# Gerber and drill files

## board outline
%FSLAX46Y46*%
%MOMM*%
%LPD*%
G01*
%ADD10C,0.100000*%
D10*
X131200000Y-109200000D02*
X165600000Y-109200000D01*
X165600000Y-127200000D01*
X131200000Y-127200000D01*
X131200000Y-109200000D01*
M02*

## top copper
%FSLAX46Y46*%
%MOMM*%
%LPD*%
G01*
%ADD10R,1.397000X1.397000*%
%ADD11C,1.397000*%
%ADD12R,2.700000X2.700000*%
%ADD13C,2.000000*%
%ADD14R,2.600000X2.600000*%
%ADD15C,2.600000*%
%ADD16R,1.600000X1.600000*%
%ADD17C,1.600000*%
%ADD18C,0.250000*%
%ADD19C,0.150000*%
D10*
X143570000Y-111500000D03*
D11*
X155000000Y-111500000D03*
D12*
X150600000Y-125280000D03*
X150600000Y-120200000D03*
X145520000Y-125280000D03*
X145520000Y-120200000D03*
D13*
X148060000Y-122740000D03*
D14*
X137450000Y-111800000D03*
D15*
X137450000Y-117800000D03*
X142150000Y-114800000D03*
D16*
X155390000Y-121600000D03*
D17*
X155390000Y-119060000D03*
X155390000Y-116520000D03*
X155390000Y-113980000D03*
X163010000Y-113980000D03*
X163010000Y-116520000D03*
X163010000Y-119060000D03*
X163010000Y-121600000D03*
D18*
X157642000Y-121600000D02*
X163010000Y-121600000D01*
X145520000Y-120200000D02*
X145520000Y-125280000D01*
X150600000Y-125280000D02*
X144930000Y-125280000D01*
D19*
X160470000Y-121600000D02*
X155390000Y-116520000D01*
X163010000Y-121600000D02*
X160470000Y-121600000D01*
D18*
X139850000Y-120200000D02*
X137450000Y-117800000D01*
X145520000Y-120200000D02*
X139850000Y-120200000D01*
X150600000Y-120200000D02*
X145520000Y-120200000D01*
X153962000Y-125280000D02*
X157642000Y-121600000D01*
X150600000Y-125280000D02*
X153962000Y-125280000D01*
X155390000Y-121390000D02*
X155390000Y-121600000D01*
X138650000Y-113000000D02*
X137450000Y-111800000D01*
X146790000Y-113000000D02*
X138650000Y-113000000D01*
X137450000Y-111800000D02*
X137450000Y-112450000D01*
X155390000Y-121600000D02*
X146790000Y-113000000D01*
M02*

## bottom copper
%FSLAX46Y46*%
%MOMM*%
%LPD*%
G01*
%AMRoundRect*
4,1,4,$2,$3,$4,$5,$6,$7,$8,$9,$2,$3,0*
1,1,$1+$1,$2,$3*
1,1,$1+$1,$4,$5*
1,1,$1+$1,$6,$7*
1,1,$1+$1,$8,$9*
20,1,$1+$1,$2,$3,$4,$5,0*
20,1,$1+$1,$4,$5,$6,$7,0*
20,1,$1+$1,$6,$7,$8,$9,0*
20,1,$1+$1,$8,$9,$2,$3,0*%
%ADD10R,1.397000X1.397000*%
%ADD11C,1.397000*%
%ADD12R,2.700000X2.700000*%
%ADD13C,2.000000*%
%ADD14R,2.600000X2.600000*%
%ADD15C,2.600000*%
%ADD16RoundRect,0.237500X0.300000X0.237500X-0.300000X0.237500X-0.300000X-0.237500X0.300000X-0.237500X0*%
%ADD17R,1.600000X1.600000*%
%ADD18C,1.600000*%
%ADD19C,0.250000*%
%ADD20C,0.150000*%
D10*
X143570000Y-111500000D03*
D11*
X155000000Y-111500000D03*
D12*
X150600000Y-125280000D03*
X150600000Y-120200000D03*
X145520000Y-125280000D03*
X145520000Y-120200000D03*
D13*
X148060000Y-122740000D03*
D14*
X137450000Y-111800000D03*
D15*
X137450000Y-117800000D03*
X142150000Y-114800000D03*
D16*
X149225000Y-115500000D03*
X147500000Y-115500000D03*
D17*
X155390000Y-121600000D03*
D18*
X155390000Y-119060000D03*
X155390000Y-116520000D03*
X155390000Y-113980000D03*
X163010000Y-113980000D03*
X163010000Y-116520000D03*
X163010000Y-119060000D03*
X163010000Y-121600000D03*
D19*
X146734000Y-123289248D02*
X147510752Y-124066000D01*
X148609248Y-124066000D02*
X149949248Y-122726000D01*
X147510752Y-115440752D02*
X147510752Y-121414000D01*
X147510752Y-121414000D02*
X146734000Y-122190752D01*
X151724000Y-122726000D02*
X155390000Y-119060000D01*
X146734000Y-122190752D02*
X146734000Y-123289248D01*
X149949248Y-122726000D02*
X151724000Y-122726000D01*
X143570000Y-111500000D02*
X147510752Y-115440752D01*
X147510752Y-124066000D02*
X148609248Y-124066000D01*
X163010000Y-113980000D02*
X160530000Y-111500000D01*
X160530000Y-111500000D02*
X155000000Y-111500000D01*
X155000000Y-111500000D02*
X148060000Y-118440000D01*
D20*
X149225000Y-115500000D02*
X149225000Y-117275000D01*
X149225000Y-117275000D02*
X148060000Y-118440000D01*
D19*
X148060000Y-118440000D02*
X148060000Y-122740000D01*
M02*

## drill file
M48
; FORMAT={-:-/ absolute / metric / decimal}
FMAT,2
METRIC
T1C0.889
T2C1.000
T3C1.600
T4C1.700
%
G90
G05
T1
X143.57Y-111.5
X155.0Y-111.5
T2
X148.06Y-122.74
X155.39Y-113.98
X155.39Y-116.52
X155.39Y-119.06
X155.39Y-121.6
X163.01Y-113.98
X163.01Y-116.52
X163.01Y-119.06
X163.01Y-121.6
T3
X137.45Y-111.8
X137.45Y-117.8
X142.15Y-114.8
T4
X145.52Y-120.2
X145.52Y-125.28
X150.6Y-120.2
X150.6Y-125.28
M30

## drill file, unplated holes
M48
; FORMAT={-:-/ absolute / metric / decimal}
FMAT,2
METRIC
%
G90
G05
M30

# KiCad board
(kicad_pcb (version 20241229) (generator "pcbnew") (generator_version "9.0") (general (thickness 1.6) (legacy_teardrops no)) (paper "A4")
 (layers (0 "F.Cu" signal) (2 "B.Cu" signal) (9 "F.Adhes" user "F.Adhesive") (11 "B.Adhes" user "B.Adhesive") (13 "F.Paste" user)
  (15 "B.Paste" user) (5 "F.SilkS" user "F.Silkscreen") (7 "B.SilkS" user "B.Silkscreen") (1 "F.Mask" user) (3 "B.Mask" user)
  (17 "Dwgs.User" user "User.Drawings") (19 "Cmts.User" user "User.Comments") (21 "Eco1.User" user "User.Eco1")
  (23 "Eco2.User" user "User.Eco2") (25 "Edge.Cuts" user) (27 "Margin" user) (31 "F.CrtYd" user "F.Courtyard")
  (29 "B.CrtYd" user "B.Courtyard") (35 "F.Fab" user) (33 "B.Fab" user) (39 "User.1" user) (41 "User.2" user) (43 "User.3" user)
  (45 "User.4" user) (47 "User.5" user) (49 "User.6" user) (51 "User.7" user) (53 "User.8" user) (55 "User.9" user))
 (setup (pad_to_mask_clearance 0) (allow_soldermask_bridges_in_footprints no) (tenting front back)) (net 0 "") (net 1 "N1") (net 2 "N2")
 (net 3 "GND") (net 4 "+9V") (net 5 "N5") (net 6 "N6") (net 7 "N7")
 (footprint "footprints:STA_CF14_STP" (layer "F.Cu") (at 143.57 111.5)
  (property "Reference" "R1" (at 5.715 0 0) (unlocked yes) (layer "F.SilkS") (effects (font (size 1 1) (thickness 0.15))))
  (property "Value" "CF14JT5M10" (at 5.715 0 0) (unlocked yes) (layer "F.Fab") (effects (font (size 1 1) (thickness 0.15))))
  (pad "1" thru_hole rect (at 0 0) (size 1.397 1.397) (drill 0.889) (layers "*.Cu" "*.Mask") (remove_unused_layers no) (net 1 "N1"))
  (pad "2" thru_hole circle (at 11.43 0) (size 1.397 1.397) (drill 0.889) (layers "*.Cu" "*.Mask") (remove_unused_layers no) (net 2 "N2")))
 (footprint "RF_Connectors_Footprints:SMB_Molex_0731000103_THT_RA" (layer "F.Cu") (at 148.06 122.74 180)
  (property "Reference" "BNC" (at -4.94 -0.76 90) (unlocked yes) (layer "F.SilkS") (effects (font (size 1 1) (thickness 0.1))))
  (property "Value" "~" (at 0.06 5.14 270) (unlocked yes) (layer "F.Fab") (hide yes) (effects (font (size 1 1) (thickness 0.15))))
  (pad "1" thru_hole rect (at -2.54 -2.54 270) (size 2.7 2.7) (drill 1.7) (layers "*.Cu" "*.Mask") (remove_unused_layers no) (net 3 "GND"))
  (pad "1" thru_hole rect (at -2.54 2.54 270) (size 2.7 2.7) (drill 1.7) (layers "*.Cu" "*.Mask") (remove_unused_layers no) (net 3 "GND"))
  (pad "1" thru_hole rect (at 2.54 -2.54 270) (size 2.7 2.7) (drill 1.7) (layers "*.Cu" "*.Mask") (remove_unused_layers no) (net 3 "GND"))
  (pad "1" thru_hole rect (at 2.54 2.54 270) (size 2.7 2.7) (drill 1.7) (layers "*.Cu" "*.Mask") (remove_unused_layers no) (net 3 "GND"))
  (pad "2" thru_hole circle (at 0 0 180) (size 2 2) (drill 1) (layers "*.Cu" "*.Mask") (remove_unused_layers no) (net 2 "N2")))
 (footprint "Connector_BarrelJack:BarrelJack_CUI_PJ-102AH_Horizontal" (layer "F.Cu") (at 137.45 111.8)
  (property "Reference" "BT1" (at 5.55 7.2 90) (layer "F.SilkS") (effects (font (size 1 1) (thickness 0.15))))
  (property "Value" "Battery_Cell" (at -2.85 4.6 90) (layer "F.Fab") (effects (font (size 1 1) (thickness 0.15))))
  (pad "1" thru_hole rect (at 0 0) (size 2.6 2.6) (drill 1.6) (layers "*.Cu" "*.Mask") (remove_unused_layers no) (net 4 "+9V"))
  (pad "2" thru_hole circle (at 0 6) (size 2.6 2.6) (drill 1.6) (layers "*.Cu" "*.Mask") (remove_unused_layers no) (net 3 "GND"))
  (pad "3" thru_hole circle (at 4.7 3) (size 2.6 2.6) (drill 1.6) (layers "*.Cu" "*.Mask") (remove_unused_layers no)))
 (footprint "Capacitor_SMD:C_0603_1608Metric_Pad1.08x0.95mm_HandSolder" (layer "B.Cu") (at 148.3625 115.5 180)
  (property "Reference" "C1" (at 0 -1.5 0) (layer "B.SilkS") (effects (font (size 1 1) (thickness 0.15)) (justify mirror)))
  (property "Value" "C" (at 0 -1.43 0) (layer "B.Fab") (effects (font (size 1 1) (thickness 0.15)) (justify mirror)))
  (pad "1" smd roundrect (at -0.8625 0 180) (size 1.075 0.95) (layers "B.Cu" "B.Mask" "B.Paste") (roundrect_rratio 0.25) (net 2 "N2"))
  (pad "2" smd roundrect (at 0.8625 0 180) (size 1.075 0.95) (layers "B.Cu" "B.Mask" "B.Paste") (roundrect_rratio 0.25) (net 1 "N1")))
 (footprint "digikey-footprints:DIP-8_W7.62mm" (layer "B.Cu") (at 155.39 121.6)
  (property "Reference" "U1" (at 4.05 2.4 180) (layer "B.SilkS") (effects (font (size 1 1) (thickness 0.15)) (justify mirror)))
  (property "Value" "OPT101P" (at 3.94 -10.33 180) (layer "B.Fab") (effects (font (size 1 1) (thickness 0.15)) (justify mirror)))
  (pad "1" thru_hole rect (at 0 0) (size 1.6 1.6) (drill 1) (layers "*.Cu" "*.Mask") (remove_unused_layers no) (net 4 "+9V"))
  (pad "2" thru_hole circle (at 0 -2.54) (size 1.6 1.6) (drill 1) (layers "*.Cu" "*.Mask") (remove_unused_layers no) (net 1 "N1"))
  (pad "3" thru_hole circle (at 0 -5.08) (size 1.6 1.6) (drill 1) (layers "*.Cu" "*.Mask") (remove_unused_layers no) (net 3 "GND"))
  (pad "4" thru_hole circle (at 0 -7.62) (size 1.6 1.6) (drill 1) (layers "*.Cu" "*.Mask") (remove_unused_layers no) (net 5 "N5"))
  (pad "5" thru_hole circle (at 7.62 -7.62) (size 1.6 1.6) (drill 1) (layers "*.Cu" "*.Mask") (remove_unused_layers no) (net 2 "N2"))
  (pad "6" thru_hole circle (at 7.62 -5.08) (size 1.6 1.6) (drill 1) (layers "*.Cu" "*.Mask") (remove_unused_layers no) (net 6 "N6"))
  (pad "7" thru_hole circle (at 7.62 -2.54) (size 1.6 1.6) (drill 1) (layers "*.Cu" "*.Mask") (remove_unused_layers no) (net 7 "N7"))
  (pad "8" thru_hole circle (at 7.62 0) (size 1.6 1.6) (drill 1) (layers "*.Cu" "*.Mask") (remove_unused_layers no) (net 3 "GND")))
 (gr_rect (start 131.2 109.2) (end 165.6 127.2) (stroke (width 0.1) (type default)) (fill no) (locked yes) (layer "Edge.Cuts"))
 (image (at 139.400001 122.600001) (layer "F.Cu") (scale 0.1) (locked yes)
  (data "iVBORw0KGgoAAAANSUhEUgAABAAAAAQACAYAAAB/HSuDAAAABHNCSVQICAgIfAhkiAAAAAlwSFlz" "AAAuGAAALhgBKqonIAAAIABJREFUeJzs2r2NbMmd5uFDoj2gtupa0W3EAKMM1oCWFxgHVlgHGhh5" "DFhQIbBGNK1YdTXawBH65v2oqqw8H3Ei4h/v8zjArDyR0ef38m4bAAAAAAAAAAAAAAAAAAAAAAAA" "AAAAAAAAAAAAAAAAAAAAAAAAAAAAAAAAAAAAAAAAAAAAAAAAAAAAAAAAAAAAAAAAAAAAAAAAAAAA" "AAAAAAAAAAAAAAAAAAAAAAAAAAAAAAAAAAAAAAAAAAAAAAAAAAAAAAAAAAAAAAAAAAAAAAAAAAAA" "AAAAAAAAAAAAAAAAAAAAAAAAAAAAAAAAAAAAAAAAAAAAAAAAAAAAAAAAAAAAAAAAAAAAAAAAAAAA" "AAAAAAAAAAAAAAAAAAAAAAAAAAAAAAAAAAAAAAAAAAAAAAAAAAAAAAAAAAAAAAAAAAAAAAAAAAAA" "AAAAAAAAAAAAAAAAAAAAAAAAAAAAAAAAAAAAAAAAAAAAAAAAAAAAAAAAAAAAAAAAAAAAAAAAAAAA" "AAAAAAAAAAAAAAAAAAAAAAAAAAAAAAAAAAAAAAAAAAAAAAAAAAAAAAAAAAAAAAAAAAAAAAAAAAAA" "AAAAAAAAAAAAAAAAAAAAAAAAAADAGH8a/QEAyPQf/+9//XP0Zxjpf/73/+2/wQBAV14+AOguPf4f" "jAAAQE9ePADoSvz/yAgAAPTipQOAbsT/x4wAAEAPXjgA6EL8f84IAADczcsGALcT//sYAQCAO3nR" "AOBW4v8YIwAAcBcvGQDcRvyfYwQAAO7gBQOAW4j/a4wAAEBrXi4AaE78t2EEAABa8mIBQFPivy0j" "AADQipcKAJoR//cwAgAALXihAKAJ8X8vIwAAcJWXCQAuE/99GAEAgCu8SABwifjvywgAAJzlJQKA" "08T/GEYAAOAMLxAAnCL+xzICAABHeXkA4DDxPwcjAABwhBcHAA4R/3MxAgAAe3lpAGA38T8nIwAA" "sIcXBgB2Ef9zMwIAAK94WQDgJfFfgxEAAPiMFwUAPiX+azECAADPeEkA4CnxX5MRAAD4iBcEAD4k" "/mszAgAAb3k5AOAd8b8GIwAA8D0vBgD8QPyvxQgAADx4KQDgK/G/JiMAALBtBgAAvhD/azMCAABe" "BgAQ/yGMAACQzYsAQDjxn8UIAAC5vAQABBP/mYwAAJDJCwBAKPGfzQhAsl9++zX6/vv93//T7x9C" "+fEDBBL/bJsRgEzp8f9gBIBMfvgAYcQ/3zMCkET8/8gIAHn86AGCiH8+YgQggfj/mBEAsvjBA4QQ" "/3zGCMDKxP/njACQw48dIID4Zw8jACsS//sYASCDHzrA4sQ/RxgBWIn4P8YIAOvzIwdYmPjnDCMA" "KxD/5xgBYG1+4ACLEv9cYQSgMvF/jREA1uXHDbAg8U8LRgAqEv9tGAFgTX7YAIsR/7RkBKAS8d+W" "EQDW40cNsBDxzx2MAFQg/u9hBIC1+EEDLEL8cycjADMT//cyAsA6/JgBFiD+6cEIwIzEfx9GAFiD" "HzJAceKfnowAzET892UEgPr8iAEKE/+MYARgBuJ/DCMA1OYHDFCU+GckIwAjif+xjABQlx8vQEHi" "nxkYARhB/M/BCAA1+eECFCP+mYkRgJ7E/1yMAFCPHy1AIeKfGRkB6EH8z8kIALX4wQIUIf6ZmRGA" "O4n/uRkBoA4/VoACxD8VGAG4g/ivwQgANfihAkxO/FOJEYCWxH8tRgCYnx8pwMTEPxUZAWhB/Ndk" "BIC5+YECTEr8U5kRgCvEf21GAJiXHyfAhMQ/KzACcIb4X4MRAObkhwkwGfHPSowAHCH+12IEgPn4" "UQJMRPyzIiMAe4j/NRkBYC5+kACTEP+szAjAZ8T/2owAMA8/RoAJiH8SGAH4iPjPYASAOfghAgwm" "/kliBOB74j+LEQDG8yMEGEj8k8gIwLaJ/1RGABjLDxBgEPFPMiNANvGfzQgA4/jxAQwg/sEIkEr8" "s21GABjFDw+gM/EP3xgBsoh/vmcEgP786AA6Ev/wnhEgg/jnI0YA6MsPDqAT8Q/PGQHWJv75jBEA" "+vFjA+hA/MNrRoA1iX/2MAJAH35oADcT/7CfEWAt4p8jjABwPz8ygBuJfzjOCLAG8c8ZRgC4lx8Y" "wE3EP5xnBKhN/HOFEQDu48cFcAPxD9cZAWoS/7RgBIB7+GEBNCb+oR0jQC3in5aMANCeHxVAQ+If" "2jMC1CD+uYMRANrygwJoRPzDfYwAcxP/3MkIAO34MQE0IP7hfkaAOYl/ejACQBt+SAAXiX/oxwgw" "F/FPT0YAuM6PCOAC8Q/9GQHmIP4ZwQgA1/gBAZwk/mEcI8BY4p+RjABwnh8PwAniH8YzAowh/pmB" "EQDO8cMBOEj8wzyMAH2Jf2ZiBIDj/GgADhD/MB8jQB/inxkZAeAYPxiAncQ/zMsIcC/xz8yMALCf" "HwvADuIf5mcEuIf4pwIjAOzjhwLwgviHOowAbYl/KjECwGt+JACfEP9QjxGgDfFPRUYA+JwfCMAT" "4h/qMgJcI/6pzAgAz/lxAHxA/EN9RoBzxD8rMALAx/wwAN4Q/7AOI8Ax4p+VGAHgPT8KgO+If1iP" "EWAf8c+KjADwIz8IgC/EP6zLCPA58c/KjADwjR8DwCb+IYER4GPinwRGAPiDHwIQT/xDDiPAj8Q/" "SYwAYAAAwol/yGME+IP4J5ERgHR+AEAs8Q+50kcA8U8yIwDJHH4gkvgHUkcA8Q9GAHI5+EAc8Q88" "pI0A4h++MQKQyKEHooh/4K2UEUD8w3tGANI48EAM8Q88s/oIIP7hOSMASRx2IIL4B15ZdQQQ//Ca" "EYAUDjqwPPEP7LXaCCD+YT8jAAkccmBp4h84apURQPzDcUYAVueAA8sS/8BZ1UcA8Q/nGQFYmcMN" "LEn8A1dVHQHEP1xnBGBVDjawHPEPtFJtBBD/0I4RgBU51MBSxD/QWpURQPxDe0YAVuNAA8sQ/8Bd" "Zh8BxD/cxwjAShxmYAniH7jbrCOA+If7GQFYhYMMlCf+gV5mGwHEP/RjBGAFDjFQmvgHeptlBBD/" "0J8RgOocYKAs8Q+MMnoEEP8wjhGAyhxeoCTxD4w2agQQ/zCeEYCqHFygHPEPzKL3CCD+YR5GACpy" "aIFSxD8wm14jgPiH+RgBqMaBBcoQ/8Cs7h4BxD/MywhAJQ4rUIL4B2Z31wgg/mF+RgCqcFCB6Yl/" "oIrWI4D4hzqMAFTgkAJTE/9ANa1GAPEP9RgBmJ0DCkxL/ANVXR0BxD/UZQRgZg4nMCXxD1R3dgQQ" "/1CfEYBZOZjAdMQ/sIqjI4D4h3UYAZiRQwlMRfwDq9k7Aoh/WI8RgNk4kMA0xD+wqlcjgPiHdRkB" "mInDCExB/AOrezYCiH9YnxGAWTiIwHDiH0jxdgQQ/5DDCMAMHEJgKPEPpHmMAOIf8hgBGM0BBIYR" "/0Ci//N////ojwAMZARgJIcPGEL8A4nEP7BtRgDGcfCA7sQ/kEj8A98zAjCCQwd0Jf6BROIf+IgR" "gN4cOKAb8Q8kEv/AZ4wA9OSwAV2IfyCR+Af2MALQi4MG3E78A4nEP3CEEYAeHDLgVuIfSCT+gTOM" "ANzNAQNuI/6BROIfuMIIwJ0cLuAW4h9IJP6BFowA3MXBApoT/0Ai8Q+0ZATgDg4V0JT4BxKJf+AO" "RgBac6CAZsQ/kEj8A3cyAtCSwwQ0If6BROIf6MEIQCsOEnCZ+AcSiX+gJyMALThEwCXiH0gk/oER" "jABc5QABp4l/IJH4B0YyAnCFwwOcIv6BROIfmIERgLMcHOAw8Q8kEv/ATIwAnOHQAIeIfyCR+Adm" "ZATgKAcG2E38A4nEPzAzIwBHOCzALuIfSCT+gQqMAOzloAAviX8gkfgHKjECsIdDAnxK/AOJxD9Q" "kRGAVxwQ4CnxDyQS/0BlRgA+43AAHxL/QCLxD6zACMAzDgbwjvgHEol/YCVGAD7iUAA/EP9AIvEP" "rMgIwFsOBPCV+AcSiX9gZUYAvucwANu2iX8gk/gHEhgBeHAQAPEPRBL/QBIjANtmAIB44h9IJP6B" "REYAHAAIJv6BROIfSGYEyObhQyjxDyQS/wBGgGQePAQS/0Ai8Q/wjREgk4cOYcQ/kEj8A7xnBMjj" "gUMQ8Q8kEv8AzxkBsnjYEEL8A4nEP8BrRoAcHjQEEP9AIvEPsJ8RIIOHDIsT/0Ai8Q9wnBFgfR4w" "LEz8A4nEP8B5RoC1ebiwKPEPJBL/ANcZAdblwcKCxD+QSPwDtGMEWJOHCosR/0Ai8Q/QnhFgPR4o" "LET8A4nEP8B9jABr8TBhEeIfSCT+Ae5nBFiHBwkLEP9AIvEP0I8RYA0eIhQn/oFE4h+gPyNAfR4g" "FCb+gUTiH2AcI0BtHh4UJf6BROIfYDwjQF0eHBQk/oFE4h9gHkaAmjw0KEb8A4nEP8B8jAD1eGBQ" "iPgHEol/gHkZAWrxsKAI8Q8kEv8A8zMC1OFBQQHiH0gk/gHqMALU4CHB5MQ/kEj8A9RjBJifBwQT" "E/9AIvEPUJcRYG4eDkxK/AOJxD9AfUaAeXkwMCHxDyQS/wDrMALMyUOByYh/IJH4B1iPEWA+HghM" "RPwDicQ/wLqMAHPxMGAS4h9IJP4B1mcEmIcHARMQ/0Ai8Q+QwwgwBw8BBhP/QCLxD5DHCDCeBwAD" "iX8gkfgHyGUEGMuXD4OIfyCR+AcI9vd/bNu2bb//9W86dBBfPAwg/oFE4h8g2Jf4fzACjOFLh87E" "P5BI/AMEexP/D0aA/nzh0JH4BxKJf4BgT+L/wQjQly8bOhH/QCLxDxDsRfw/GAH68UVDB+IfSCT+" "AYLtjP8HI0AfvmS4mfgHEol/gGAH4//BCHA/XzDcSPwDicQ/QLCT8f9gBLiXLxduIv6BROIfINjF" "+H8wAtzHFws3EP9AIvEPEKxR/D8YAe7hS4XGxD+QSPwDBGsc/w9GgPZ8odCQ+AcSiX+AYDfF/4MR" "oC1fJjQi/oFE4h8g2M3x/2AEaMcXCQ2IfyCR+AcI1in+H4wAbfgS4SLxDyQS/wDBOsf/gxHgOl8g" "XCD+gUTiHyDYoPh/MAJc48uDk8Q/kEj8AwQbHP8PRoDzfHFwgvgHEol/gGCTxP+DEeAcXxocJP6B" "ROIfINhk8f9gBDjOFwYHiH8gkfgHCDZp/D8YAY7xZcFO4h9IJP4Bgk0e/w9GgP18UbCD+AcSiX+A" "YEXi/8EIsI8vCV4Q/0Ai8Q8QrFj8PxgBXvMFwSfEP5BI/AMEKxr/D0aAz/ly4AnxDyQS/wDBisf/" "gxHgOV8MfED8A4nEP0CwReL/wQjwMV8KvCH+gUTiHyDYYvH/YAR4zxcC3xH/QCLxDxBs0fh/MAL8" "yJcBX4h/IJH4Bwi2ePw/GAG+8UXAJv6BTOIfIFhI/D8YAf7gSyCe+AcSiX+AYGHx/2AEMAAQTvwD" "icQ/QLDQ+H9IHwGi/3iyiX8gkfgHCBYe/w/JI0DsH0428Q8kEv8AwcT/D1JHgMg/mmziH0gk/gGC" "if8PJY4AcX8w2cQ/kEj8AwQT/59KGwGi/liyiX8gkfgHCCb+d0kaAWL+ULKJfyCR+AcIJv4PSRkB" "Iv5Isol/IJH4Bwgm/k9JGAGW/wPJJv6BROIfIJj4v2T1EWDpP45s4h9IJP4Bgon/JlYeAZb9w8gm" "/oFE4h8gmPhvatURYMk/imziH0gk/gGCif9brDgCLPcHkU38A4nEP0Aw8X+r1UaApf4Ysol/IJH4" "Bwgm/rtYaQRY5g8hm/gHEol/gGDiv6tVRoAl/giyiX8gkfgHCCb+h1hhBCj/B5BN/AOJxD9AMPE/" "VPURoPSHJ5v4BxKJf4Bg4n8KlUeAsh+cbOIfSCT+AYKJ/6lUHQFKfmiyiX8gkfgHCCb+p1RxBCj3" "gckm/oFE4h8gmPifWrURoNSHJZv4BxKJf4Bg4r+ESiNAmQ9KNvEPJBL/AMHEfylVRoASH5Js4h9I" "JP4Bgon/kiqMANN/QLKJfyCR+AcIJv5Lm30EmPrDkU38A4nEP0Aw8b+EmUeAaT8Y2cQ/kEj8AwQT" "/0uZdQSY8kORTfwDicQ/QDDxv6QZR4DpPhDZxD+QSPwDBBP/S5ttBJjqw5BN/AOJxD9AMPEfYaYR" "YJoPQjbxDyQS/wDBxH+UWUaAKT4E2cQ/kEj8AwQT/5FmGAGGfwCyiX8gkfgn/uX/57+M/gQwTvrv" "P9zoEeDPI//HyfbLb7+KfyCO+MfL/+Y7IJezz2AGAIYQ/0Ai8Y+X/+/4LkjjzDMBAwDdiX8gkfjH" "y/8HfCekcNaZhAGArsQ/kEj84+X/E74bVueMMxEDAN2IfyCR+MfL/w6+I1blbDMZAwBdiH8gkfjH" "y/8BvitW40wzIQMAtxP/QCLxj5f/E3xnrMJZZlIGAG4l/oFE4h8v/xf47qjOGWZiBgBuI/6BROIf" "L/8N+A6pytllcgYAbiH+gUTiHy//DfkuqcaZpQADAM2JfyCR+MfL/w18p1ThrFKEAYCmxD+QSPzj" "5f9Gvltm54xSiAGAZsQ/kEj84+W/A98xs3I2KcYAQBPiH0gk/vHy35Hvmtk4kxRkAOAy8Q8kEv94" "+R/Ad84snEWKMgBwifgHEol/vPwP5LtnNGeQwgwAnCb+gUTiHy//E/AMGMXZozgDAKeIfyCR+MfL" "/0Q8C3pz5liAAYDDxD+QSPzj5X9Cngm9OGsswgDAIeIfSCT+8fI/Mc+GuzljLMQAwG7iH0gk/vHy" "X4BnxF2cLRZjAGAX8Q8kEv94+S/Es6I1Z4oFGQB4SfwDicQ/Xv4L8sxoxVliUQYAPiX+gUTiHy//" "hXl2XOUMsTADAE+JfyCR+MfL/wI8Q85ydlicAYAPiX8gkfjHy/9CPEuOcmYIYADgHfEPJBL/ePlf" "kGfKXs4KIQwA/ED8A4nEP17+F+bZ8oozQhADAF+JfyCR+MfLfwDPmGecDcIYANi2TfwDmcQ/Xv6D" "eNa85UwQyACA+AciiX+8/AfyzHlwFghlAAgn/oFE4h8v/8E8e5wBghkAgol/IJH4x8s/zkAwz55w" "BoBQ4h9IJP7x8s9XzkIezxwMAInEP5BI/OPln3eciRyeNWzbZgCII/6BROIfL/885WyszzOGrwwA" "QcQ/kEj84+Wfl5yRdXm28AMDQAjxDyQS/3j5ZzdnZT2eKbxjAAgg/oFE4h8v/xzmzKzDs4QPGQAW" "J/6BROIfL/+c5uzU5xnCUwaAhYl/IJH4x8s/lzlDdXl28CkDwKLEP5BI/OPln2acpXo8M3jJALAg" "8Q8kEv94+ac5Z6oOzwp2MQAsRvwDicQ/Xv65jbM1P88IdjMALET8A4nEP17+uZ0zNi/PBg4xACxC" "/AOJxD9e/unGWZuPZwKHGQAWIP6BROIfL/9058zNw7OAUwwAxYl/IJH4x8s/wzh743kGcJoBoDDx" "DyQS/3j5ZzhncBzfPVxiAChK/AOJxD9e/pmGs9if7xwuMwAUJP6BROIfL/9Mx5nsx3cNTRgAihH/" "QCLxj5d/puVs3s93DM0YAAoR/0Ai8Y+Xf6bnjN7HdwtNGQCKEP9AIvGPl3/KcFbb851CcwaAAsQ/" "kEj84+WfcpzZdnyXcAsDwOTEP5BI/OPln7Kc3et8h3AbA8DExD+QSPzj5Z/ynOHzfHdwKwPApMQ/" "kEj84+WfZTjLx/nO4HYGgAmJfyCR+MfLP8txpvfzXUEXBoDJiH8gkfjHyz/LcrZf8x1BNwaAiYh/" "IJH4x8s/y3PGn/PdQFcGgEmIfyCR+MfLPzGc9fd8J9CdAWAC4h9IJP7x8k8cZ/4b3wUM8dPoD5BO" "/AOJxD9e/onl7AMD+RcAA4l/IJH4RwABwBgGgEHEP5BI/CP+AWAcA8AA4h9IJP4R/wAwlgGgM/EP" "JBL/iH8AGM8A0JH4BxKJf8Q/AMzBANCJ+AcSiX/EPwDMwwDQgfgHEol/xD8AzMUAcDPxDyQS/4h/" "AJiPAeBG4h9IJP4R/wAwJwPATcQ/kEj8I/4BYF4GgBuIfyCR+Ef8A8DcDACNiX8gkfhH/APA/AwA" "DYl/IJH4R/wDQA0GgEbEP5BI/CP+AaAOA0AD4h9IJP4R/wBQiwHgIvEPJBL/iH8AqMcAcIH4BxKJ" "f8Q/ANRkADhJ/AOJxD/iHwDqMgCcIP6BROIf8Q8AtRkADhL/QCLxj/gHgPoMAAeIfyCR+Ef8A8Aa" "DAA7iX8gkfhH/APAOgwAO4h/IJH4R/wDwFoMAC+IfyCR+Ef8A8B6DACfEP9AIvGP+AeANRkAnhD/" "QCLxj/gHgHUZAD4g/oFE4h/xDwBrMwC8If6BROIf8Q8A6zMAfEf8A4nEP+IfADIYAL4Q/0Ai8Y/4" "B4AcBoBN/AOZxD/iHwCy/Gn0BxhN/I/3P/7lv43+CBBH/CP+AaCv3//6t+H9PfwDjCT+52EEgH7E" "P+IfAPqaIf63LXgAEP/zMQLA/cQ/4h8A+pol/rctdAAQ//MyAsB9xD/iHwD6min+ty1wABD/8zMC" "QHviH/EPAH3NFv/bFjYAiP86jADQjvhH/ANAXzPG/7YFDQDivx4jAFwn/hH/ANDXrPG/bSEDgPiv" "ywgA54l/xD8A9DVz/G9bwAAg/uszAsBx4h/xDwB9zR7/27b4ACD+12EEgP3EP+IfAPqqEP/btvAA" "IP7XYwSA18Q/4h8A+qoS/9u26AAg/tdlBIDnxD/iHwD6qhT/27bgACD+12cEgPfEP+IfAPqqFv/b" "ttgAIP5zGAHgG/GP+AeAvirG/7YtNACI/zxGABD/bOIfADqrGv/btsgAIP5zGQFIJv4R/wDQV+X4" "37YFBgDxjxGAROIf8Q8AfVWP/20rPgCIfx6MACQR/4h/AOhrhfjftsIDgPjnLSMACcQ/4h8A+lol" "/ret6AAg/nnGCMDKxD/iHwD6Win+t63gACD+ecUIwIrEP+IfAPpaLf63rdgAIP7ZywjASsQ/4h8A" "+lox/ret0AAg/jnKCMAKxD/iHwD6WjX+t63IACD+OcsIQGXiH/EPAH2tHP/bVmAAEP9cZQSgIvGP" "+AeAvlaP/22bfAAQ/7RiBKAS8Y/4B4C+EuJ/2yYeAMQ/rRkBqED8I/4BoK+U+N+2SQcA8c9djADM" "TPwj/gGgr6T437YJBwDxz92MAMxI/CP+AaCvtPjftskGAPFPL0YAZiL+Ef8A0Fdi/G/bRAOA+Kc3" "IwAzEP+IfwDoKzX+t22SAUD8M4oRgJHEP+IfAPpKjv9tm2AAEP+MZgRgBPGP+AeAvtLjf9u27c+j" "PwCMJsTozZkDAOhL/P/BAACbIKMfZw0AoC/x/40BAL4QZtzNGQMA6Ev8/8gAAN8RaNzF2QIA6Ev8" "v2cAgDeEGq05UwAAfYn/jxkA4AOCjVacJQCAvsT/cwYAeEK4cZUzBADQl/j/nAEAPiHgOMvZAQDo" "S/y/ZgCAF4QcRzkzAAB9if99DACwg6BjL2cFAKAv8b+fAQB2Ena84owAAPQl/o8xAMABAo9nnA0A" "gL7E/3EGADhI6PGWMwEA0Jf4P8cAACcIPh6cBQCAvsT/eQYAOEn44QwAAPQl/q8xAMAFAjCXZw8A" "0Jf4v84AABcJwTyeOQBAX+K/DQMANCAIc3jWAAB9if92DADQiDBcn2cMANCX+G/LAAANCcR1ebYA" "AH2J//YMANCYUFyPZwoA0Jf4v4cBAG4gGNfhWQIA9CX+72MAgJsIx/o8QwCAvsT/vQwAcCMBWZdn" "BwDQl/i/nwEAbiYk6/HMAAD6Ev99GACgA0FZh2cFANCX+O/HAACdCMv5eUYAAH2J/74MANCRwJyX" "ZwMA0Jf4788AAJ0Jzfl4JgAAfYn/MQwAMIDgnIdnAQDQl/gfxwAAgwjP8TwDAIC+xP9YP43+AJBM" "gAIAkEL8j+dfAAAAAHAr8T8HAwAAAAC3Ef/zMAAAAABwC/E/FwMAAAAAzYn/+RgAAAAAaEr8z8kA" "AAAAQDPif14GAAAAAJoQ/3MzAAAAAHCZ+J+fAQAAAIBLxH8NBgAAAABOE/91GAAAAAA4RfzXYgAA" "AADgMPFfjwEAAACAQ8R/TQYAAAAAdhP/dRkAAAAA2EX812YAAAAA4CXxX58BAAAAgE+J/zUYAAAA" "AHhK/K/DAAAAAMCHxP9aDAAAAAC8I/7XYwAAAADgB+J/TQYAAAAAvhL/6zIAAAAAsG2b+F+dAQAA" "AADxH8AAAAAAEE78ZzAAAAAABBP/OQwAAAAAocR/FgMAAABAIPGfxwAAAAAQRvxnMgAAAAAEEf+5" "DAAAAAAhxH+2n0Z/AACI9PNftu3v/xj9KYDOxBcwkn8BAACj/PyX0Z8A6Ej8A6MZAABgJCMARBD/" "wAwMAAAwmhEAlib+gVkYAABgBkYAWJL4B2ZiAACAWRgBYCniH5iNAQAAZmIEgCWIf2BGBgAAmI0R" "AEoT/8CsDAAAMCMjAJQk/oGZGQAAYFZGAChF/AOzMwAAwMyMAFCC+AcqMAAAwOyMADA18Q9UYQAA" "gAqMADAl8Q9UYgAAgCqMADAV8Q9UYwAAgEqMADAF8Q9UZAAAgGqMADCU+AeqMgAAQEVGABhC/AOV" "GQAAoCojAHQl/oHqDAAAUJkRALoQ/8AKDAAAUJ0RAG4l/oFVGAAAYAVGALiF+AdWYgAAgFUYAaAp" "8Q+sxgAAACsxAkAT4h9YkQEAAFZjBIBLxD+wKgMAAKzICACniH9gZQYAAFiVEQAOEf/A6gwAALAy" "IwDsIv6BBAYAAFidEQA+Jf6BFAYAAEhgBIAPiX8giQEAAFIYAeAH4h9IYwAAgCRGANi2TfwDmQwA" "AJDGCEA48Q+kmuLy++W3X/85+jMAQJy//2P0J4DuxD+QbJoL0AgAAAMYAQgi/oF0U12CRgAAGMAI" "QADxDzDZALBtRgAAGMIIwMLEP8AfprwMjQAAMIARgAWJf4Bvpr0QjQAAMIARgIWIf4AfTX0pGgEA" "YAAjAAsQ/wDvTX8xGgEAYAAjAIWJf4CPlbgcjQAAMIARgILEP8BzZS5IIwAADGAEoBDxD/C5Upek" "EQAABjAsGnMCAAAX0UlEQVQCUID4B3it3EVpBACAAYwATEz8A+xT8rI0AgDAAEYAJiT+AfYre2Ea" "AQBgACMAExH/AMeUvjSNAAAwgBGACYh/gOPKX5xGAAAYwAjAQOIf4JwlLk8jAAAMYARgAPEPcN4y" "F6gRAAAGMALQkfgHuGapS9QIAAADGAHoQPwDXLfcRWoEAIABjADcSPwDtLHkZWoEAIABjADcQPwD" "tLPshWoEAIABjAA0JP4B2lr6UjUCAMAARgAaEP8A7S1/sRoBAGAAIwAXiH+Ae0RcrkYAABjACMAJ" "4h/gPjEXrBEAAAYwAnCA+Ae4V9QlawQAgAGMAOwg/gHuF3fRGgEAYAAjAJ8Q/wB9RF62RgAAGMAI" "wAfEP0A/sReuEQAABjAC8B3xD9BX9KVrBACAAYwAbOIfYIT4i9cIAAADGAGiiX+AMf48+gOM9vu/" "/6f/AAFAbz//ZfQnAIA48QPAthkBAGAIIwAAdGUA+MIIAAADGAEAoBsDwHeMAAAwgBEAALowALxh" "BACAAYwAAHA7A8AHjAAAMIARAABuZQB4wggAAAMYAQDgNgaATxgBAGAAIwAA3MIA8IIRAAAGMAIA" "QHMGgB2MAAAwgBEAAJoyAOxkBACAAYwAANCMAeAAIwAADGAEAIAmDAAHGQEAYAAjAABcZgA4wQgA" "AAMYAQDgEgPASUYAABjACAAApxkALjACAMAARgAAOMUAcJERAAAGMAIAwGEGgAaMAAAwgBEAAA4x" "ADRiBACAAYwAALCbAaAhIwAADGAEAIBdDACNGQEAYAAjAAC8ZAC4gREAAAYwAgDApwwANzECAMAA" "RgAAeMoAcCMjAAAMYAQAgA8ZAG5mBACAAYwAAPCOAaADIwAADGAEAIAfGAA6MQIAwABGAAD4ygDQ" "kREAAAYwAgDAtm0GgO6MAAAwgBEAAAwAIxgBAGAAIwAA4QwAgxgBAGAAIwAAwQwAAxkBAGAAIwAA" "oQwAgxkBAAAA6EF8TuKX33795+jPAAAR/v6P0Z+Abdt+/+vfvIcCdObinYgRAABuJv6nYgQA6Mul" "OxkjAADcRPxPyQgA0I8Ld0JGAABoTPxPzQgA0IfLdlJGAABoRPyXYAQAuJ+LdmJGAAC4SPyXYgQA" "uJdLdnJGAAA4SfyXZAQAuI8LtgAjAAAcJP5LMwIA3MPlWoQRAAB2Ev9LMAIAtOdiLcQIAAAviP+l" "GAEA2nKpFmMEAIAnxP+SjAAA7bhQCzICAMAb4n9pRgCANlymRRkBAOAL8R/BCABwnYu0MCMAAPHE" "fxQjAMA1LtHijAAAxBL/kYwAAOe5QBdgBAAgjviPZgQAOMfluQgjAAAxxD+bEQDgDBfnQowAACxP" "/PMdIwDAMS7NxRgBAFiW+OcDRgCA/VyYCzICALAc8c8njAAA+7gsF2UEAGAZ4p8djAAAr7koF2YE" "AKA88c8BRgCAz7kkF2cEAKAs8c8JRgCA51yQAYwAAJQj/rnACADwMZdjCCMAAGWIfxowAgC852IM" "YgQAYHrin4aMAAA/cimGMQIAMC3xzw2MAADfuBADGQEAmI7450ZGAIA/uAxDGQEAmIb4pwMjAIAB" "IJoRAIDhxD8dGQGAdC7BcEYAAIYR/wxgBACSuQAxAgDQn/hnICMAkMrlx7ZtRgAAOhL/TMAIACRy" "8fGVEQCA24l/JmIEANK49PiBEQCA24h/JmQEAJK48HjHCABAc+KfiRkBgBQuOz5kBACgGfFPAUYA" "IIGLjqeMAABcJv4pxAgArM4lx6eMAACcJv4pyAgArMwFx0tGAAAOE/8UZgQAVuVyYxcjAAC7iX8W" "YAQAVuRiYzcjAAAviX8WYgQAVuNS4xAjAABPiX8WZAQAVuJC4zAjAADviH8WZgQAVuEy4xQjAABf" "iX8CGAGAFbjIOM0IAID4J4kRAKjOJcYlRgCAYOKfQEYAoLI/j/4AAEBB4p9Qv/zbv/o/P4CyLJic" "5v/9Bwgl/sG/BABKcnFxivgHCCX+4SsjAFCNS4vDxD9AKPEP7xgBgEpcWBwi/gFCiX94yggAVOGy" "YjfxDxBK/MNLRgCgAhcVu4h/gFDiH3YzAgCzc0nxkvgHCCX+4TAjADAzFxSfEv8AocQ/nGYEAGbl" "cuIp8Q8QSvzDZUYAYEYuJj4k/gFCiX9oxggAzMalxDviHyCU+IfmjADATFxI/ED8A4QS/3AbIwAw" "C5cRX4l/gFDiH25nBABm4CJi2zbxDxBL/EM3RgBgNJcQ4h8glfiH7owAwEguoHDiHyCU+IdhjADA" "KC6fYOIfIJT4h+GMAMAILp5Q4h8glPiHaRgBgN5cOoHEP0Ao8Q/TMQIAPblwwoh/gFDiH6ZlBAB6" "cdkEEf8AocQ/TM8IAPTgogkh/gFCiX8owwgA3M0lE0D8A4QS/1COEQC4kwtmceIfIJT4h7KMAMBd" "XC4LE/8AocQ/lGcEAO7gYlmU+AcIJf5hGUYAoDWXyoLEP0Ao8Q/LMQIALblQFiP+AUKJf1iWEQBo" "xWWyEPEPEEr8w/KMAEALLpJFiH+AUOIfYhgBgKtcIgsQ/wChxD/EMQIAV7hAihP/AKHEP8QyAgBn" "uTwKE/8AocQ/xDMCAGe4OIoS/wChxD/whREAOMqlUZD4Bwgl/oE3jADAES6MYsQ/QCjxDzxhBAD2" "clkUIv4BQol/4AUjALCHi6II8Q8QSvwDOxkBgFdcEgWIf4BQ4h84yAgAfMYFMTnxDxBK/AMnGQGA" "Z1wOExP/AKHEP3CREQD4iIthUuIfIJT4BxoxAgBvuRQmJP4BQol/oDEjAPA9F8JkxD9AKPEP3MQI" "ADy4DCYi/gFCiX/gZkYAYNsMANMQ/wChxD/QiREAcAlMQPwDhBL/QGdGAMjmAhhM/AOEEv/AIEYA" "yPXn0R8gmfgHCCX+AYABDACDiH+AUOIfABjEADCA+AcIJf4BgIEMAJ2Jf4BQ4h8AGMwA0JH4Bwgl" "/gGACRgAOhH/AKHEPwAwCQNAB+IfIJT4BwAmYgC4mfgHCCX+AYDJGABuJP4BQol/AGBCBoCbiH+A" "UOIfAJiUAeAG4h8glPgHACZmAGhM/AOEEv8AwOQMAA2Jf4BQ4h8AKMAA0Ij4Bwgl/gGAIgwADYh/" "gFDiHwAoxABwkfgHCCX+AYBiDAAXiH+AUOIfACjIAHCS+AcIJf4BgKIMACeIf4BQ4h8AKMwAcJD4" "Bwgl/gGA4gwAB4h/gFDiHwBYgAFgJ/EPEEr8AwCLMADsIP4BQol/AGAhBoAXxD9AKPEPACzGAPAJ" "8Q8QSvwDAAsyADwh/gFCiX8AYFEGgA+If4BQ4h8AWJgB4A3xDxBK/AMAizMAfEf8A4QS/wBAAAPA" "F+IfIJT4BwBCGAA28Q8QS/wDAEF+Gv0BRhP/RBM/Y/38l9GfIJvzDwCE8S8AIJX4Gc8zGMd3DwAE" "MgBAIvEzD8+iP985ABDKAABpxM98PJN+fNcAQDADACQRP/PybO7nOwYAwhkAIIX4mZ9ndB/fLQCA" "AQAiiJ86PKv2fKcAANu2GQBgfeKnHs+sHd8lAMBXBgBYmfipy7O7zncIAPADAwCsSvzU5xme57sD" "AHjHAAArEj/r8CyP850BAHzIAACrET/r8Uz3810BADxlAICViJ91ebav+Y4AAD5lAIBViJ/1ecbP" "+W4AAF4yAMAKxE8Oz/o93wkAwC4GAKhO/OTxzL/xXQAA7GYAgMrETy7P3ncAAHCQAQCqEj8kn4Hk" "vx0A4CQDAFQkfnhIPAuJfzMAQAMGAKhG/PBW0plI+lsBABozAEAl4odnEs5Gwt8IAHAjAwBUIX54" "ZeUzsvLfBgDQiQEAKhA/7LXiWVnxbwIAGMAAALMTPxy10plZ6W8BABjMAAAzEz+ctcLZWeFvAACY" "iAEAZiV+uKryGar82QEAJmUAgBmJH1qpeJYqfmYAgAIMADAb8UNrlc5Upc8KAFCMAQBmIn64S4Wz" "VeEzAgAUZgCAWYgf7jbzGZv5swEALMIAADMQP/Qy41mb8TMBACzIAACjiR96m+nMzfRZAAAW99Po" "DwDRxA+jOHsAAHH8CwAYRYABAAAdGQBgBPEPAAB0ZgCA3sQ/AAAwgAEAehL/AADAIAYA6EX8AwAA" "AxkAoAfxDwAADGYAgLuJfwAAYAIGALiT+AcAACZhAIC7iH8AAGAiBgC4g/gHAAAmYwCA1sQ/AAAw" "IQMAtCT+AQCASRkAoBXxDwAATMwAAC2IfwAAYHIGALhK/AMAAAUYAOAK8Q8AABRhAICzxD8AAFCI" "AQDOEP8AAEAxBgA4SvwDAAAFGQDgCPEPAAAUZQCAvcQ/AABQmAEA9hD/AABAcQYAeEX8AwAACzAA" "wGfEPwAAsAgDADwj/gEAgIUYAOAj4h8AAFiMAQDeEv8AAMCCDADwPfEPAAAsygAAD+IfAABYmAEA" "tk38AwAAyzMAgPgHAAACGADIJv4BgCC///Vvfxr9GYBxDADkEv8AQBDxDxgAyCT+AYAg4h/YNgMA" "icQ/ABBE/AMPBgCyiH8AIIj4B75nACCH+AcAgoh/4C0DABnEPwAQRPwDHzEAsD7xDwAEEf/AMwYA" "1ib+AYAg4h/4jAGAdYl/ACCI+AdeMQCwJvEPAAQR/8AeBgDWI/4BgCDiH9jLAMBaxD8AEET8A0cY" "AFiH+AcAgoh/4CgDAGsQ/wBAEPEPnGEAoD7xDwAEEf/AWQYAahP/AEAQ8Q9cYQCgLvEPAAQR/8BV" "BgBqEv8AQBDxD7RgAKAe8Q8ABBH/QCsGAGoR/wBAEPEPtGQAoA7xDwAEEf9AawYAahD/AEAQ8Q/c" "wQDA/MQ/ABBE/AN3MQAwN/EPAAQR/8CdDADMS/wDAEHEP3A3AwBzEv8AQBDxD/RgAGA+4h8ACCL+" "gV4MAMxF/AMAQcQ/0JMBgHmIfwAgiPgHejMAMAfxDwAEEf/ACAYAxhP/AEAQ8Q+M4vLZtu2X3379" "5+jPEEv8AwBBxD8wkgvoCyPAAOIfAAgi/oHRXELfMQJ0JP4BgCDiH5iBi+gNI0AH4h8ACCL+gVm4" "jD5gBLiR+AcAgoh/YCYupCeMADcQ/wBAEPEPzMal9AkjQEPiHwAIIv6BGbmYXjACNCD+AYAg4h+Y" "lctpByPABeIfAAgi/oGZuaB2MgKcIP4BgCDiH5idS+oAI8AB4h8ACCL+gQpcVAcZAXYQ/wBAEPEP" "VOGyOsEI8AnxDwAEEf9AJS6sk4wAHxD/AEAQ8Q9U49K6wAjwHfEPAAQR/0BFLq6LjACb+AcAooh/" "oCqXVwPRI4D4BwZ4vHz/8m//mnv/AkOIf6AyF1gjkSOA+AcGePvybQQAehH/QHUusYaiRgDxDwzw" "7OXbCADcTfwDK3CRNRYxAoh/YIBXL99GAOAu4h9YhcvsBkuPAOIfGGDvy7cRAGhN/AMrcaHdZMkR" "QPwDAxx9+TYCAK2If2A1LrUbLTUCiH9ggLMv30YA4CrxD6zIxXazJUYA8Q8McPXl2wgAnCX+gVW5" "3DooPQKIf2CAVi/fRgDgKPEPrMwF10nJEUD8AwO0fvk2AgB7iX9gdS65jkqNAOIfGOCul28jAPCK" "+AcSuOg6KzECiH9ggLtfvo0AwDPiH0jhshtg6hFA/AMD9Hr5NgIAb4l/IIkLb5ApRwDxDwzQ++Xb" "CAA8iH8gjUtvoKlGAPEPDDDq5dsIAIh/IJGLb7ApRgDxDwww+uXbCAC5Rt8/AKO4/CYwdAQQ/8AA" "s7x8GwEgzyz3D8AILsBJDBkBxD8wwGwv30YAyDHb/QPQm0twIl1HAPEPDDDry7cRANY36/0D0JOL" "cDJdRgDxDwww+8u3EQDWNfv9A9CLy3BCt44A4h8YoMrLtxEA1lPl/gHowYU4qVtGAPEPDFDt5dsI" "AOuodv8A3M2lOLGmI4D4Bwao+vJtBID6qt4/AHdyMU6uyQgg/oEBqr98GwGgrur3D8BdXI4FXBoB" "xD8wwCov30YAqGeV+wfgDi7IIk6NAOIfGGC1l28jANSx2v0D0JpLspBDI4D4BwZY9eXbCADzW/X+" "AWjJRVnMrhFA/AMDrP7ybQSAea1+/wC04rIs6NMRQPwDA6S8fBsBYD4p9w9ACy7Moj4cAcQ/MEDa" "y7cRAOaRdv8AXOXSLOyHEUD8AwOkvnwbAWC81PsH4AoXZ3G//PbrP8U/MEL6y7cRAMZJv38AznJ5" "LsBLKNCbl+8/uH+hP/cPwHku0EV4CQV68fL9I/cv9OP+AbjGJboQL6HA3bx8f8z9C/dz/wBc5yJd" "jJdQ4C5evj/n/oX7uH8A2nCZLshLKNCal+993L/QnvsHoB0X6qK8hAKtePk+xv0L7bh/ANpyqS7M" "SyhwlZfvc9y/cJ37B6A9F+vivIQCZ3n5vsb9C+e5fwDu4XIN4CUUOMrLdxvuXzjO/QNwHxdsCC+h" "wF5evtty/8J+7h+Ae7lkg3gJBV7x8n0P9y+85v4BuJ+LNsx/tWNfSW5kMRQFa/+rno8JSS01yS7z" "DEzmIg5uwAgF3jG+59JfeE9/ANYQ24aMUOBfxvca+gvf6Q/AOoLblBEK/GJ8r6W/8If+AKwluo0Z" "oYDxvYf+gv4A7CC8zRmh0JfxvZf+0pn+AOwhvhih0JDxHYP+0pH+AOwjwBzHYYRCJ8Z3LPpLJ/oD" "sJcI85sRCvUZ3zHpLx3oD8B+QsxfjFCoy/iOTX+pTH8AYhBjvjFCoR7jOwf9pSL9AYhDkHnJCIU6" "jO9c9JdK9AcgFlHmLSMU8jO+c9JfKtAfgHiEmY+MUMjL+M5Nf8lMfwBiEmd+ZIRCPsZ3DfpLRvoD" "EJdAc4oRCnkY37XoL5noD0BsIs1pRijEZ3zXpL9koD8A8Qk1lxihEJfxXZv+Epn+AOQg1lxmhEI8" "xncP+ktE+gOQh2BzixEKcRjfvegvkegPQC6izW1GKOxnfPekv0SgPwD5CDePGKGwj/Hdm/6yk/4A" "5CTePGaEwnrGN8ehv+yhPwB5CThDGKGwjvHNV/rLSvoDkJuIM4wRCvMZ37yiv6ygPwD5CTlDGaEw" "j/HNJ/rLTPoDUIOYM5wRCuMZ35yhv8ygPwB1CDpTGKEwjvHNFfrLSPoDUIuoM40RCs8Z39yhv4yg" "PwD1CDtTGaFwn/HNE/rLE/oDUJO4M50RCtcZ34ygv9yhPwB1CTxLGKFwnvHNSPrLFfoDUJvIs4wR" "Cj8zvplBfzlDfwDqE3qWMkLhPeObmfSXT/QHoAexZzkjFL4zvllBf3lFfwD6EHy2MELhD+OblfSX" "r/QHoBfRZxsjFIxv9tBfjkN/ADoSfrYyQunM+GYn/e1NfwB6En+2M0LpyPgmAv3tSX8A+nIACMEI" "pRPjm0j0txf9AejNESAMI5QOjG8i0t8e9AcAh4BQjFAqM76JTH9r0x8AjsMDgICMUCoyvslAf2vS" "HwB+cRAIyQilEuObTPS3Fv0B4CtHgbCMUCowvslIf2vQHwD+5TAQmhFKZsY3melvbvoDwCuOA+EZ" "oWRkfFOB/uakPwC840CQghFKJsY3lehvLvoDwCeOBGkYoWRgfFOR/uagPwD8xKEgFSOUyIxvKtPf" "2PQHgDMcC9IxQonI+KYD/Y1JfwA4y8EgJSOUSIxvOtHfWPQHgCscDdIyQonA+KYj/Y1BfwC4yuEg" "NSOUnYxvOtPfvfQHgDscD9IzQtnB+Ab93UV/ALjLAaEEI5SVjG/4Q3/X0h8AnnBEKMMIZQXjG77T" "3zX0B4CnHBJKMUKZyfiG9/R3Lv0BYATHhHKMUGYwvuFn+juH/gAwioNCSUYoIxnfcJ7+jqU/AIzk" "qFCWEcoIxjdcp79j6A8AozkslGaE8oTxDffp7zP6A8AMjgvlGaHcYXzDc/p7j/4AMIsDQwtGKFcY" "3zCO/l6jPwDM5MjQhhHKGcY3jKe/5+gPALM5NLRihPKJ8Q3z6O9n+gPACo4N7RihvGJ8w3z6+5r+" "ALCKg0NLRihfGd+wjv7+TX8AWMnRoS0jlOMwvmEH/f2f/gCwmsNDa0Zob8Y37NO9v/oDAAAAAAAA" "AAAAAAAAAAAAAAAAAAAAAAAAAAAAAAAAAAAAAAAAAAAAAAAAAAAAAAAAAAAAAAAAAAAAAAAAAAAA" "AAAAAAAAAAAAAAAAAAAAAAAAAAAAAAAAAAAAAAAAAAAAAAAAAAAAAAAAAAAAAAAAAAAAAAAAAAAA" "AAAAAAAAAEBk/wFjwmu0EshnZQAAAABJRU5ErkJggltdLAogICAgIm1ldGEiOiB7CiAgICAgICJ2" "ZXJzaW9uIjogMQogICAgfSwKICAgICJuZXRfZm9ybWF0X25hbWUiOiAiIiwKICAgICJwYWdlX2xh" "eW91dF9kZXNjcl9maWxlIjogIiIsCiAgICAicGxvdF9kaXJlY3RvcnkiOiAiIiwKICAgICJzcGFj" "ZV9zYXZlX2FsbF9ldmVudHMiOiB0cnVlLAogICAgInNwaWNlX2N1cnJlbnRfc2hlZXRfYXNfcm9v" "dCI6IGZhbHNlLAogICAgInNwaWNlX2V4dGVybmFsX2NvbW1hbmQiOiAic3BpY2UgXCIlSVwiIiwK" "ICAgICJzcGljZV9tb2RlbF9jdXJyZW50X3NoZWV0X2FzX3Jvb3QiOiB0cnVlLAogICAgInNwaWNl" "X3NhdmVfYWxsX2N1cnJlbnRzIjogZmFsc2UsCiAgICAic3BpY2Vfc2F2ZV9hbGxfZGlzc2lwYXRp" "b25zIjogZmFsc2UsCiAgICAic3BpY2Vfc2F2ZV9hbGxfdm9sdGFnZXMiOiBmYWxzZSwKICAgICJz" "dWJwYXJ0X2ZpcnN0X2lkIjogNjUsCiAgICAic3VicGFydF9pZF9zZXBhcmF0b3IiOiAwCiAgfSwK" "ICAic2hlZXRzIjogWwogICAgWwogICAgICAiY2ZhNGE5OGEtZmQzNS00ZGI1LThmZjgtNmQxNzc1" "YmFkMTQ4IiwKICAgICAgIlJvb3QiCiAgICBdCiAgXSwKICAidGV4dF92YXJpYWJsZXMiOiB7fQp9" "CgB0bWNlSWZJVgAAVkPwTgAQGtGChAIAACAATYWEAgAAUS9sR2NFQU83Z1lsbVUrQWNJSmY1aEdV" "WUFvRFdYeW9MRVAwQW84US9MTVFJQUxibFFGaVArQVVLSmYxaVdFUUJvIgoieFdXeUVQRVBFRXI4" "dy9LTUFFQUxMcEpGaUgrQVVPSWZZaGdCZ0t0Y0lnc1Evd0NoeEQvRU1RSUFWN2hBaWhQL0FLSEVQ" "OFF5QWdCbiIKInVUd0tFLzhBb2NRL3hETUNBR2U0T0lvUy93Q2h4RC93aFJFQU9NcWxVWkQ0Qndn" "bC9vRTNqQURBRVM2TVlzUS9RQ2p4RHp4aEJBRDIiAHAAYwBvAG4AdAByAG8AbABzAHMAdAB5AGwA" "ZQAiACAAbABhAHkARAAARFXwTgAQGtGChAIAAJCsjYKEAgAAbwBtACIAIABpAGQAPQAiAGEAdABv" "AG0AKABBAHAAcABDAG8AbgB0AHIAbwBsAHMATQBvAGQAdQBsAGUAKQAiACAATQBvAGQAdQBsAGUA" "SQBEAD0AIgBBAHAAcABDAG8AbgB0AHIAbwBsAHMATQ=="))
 (segment (start 157.642 121.6) (end 163.01 121.6) (width 0.25) (layer "F.Cu") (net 3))
 (segment (start 145.52 120.2) (end 145.52 125.28) (width 0.25) (layer "F.Cu") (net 3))
 (segment (start 150.6 125.28) (end 144.93 125.28) (width 0.25) (layer "F.Cu") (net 3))
 (segment (start 160.47 121.6) (end 155.39 116.52) (width 0.15) (layer "F.Cu") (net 3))
 (segment (start 163.01 121.6) (end 160.47 121.6) (width 0.15) (layer "F.Cu") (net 3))
 (segment (start 139.85 120.2) (end 137.45 117.8) (width 0.25) (layer "F.Cu") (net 3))
 (segment (start 145.52 120.2) (end 139.85 120.2) (width 0.25) (layer "F.Cu") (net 3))
 (segment (start 150.6 120.2) (end 145.52 120.2) (width 0.25) (layer "F.Cu") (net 3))
 (segment (start 153.962 125.28) (end 157.642 121.6) (width 0.25) (layer "F.Cu") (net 3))
 (segment (start 150.6 125.28) (end 153.962 125.28) (width 0.25) (layer "F.Cu") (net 3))
 (segment (start 155.39 121.39) (end 155.39 121.6) (width 0.25) (layer "F.Cu") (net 4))
 (segment (start 138.65 113) (end 137.45 111.8) (width 0.25) (layer "F.Cu") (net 4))
 (segment (start 146.79 113) (end 138.65 113) (width 0.25) (layer "F.Cu") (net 4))
 (segment (start 137.45 111.8) (end 137.45 112.45) (width 0.25) (layer "F.Cu") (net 4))
 (segment (start 155.39 121.6) (end 146.79 113) (width 0.25) (layer "F.Cu") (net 4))
 (segment (start 146.734 123.289248) (end 147.510752 124.066) (width 0.25) (layer "B.Cu") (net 1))
 (segment (start 148.609248 124.066) (end 149.949248 122.726) (width 0.25) (layer "B.Cu") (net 1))
 (segment (start 147.510752 115.440752) (end 147.510752 121.414) (width 0.25) (layer "B.Cu") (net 1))
 (segment (start 147.510752 121.414) (end 146.734 122.190752) (width 0.25) (layer "B.Cu") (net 1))
 (segment (start 151.724 122.726) (end 155.39 119.06) (width 0.25) (layer "B.Cu") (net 1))
 (segment (start 146.734 122.190752) (end 146.734 123.289248) (width 0.25) (layer "B.Cu") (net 1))
 (segment (start 149.949248 122.726) (end 151.724 122.726) (width 0.25) (layer "B.Cu") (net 1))
 (segment (start 143.57 111.5) (end 147.510752 115.440752) (width 0.25) (layer "B.Cu") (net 1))
 (segment (start 147.510752 124.066) (end 148.609248 124.066) (width 0.25) (layer "B.Cu") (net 1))
 (segment (start 163.01 113.98) (end 160.53 111.5) (width 0.25) (layer "B.Cu") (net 2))
 (segment (start 160.53 111.5) (end 155 111.5) (width 0.25) (layer "B.Cu") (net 2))
 (segment (start 155 111.5) (end 148.06 118.44) (width 0.25) (layer "B.Cu") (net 2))
 (segment (start 149.225 115.5) (end 149.225 117.275) (width 0.15) (layer "B.Cu") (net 2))
 (segment (start 149.225 117.275) (end 148.06 118.44) (width 0.15) (layer "B.Cu") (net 2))
 (segment (start 148.06 118.44) (end 148.06 122.74) (width 0.25) (layer "B.Cu") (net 2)))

